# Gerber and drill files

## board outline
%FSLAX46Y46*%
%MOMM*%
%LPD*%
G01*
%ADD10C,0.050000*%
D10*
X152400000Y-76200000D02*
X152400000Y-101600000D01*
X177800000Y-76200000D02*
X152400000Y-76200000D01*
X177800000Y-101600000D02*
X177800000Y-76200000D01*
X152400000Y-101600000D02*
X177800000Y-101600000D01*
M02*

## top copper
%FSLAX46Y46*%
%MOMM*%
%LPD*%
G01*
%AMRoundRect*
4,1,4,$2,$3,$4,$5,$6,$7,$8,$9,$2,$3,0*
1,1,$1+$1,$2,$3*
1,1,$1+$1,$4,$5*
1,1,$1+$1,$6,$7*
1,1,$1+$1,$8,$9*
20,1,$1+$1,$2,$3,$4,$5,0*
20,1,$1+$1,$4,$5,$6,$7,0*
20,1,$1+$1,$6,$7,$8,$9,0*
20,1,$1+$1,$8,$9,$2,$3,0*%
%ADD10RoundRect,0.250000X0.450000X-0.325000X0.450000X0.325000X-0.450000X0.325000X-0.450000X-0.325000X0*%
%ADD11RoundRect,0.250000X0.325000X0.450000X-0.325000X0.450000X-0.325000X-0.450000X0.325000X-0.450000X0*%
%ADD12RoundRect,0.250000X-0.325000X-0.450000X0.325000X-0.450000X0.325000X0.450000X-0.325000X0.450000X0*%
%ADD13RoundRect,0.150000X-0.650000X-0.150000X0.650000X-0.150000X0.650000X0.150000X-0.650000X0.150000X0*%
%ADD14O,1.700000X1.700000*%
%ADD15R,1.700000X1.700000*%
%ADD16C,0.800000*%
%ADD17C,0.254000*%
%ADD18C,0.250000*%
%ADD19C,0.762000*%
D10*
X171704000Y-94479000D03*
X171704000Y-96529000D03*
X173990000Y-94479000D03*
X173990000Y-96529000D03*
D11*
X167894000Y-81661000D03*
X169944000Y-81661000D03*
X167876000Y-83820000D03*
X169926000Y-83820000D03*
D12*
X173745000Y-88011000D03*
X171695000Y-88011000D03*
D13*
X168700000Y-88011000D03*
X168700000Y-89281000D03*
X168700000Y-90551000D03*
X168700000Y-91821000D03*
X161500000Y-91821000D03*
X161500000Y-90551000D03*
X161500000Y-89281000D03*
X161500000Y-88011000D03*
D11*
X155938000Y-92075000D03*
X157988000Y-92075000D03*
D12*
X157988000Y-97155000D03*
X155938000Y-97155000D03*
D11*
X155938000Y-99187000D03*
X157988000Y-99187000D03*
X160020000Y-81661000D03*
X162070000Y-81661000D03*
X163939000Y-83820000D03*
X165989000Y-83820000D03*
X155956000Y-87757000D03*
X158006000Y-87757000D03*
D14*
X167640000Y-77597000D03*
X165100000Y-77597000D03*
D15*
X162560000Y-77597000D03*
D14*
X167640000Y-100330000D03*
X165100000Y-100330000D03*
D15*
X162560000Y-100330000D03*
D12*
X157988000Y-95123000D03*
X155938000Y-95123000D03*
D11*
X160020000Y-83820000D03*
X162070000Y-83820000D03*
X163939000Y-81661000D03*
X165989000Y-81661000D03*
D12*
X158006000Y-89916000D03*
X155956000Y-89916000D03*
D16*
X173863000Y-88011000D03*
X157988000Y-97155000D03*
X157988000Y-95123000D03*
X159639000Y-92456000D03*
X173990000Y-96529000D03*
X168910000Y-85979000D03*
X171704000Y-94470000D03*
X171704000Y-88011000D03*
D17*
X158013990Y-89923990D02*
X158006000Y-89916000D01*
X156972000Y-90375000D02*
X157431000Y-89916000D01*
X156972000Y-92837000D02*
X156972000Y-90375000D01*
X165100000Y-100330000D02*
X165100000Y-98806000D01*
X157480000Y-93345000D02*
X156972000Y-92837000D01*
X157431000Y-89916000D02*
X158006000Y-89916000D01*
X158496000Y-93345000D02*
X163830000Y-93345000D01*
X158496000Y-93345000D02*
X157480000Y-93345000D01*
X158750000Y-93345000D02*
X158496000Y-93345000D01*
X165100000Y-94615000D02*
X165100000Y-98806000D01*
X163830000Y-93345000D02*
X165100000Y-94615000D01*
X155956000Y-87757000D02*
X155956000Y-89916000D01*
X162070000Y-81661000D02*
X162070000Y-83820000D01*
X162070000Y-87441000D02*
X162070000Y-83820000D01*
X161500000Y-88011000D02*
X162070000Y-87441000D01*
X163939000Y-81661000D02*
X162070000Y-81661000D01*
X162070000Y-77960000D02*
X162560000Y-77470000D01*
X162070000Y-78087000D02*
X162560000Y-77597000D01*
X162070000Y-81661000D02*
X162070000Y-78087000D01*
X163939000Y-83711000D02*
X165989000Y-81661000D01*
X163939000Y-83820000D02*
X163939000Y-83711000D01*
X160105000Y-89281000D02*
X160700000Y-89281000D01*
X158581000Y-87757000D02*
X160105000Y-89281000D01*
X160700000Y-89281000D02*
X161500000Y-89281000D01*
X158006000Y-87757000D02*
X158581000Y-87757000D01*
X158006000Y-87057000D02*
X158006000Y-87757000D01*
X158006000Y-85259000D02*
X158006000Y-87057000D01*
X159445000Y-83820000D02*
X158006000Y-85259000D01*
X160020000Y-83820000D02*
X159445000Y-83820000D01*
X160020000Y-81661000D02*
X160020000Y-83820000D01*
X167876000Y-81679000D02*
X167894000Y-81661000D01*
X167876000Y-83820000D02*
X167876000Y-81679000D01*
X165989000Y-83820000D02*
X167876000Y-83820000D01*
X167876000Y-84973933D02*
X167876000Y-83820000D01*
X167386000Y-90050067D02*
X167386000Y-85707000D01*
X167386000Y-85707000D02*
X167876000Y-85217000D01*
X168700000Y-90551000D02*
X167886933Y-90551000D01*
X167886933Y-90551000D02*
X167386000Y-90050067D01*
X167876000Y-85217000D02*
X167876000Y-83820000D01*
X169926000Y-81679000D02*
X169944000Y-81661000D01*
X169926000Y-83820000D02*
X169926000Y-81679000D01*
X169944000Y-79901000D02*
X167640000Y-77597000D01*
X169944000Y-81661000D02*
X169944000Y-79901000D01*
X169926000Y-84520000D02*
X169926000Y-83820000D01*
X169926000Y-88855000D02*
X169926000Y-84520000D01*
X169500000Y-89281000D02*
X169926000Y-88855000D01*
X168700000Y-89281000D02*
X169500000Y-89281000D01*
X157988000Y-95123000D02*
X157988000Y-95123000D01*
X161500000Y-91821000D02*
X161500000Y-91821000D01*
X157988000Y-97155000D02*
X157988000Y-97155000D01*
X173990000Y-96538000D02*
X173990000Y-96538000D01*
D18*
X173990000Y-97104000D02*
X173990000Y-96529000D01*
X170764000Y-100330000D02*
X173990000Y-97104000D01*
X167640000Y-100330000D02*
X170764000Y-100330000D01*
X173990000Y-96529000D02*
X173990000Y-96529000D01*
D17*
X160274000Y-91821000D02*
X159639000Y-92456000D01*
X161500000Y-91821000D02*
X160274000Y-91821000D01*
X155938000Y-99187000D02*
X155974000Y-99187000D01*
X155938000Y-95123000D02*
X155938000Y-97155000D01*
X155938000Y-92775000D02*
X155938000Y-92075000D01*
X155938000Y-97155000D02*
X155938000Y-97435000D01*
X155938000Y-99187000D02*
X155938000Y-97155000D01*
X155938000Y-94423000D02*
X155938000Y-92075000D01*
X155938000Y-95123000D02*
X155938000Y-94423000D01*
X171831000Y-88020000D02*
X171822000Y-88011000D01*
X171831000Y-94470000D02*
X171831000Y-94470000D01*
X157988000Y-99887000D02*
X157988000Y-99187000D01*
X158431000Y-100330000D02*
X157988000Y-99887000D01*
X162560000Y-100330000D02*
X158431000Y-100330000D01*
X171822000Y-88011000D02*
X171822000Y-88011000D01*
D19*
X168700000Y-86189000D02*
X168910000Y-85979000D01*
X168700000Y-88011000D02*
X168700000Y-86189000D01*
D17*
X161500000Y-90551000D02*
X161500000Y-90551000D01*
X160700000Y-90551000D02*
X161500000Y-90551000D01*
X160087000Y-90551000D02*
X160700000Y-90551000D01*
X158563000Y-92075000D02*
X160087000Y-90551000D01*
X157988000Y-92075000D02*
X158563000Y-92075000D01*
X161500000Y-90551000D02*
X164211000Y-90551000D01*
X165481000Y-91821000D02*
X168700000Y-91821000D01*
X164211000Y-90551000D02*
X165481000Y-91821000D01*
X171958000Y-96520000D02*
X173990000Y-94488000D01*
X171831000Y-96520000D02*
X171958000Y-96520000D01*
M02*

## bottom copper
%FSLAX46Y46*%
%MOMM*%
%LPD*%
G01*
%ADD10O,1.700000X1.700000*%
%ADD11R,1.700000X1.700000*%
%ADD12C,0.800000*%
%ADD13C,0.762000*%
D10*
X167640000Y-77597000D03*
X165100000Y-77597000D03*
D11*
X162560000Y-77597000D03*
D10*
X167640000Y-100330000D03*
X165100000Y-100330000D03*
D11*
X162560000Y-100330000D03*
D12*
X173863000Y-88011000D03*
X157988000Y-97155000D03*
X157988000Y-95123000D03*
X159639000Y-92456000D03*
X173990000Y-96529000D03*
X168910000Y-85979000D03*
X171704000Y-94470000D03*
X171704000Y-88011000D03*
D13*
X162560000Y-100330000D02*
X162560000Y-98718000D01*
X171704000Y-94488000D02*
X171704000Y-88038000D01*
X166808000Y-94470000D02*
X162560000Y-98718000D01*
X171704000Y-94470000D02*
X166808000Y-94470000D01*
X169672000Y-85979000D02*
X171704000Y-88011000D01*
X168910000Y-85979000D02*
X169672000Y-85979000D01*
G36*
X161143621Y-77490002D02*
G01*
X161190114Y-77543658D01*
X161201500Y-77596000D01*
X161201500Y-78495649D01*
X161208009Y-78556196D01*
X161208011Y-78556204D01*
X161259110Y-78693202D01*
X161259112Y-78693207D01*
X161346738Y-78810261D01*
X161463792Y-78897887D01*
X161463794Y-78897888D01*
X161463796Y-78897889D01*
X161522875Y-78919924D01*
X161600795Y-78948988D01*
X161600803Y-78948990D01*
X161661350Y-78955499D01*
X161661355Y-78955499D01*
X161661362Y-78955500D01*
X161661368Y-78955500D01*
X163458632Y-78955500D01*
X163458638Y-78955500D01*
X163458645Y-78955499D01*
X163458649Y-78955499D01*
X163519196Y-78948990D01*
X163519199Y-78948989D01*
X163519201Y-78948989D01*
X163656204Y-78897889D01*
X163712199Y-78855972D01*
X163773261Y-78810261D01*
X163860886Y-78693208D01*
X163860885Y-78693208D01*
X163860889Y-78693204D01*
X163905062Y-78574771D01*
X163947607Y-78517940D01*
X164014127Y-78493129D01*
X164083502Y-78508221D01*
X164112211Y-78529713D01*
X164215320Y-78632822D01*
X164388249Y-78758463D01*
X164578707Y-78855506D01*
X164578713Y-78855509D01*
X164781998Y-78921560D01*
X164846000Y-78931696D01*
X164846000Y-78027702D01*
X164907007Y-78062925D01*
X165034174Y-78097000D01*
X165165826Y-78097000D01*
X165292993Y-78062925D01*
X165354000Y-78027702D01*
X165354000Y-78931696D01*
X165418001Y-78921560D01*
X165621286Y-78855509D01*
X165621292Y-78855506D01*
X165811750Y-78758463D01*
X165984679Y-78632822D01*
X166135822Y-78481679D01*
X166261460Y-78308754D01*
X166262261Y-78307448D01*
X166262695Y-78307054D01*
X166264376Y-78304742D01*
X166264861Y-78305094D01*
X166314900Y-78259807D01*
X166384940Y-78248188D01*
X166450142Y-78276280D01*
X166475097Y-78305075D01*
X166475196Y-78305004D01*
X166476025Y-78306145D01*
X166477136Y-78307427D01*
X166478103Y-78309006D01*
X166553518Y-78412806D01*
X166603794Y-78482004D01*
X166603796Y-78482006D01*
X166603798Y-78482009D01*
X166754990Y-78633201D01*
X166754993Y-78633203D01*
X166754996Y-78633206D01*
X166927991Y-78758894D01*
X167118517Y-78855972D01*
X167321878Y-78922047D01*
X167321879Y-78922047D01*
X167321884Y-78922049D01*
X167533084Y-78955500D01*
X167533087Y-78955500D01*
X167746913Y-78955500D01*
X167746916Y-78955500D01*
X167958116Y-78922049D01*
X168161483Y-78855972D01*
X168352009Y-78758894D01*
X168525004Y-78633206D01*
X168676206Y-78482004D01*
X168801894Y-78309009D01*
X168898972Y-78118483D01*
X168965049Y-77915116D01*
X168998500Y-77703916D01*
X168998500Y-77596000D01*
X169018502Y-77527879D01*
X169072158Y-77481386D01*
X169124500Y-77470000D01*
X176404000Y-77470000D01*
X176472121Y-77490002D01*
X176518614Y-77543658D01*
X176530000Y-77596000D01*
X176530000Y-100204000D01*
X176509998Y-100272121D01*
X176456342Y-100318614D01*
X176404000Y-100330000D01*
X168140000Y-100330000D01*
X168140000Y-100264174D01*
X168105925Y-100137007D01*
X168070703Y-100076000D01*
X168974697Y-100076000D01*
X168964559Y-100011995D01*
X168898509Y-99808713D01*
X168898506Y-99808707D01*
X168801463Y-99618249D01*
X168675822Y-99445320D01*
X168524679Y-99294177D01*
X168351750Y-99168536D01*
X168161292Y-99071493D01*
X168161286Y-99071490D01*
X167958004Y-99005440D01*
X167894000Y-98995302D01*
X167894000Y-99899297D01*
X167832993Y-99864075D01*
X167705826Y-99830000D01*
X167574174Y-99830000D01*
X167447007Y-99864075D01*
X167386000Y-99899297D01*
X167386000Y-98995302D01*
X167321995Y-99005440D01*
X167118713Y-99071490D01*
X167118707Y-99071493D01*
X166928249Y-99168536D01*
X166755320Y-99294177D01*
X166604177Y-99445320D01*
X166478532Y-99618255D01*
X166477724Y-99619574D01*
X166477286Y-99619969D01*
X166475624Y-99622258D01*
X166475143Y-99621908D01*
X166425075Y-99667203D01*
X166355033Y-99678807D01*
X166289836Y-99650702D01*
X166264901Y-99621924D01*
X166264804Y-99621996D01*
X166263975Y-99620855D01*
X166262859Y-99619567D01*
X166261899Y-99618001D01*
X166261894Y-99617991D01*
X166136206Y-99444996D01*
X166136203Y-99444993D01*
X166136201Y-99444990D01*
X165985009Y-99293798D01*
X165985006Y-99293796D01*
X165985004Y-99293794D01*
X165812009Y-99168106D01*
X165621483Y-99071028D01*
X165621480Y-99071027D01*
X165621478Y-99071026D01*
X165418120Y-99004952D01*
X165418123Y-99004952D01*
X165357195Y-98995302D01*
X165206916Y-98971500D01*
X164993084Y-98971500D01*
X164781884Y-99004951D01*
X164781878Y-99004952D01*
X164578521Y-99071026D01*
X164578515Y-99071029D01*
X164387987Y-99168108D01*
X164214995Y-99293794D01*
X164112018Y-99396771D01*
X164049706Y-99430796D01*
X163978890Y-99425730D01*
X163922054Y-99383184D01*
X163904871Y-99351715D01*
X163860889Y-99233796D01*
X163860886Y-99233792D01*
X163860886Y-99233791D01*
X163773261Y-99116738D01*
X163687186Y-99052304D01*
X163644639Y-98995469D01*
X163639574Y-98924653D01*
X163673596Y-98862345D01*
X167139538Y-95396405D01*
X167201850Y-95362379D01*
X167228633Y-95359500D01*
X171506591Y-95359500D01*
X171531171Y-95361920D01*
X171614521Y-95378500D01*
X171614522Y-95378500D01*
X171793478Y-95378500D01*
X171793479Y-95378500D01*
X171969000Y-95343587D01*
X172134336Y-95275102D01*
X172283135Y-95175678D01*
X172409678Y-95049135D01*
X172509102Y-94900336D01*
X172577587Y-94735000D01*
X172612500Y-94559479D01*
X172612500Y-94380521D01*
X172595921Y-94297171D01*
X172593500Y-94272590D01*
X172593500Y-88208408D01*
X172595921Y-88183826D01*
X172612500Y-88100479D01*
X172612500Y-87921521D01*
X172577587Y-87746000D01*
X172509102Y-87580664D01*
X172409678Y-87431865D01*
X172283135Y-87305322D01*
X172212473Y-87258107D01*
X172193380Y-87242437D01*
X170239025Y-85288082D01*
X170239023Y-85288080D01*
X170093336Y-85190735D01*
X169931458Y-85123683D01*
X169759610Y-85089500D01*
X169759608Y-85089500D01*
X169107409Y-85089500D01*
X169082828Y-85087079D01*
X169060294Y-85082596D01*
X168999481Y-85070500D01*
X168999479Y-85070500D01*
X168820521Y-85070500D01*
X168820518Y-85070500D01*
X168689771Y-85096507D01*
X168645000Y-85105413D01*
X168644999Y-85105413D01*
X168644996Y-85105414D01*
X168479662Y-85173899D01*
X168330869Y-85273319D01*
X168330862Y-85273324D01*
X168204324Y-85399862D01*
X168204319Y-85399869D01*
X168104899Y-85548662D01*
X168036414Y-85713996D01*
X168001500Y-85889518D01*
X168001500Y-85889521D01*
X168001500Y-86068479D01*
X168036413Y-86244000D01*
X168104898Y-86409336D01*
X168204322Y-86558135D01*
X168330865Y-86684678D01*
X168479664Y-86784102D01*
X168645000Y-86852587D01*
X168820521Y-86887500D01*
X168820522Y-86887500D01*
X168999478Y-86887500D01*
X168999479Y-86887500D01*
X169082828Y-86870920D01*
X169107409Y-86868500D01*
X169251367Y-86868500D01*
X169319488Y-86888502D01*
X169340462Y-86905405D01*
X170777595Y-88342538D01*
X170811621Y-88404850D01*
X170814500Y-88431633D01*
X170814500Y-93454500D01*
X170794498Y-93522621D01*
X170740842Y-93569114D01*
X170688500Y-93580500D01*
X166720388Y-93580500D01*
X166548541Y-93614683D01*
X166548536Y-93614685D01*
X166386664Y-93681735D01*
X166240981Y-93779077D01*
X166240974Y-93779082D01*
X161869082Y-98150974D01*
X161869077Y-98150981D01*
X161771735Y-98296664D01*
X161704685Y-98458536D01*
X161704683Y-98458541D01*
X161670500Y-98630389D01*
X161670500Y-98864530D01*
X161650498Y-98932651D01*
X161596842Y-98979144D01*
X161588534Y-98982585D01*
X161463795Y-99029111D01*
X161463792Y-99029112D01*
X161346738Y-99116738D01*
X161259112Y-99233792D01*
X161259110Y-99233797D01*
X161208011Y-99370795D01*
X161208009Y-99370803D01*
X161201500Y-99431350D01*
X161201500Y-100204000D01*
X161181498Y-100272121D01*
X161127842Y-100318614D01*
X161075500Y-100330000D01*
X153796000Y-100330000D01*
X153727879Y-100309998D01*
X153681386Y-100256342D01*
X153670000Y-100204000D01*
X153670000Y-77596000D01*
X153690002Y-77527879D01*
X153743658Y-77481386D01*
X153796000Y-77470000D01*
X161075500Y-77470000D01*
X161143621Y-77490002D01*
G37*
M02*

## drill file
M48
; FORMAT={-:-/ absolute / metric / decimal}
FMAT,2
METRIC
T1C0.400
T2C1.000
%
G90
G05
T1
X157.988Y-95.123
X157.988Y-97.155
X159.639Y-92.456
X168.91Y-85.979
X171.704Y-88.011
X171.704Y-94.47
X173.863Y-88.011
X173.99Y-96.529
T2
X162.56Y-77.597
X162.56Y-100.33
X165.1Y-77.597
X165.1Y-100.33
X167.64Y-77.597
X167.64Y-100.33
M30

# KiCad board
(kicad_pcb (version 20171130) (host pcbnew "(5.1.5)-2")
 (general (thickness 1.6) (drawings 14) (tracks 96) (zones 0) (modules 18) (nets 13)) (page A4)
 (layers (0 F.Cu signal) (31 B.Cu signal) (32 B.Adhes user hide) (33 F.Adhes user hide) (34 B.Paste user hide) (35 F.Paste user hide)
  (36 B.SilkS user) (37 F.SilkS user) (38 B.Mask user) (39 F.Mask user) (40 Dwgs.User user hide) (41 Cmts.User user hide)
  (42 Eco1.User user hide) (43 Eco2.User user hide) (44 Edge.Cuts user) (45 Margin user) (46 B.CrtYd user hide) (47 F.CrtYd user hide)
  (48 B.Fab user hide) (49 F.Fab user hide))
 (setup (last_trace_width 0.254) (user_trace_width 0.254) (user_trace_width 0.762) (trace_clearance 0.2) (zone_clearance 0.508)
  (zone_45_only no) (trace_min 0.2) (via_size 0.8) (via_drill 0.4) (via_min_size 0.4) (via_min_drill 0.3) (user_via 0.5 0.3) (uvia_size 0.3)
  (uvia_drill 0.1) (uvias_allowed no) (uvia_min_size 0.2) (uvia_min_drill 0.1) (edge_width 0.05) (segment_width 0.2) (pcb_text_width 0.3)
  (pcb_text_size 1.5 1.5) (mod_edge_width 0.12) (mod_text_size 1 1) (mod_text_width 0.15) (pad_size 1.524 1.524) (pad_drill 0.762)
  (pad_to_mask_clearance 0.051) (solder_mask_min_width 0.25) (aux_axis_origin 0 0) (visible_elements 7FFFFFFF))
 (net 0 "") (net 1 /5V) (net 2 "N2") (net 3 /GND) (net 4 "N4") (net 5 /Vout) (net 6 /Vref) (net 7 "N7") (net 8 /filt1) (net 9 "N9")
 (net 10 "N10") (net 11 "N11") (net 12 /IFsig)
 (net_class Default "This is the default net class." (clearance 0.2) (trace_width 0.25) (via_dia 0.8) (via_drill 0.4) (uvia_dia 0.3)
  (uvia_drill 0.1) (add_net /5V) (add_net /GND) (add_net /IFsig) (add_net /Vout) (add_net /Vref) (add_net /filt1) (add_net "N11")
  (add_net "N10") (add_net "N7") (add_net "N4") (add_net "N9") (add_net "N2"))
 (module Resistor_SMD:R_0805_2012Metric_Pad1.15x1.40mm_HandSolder (layer F.Cu) (at 171.704 95.504 90)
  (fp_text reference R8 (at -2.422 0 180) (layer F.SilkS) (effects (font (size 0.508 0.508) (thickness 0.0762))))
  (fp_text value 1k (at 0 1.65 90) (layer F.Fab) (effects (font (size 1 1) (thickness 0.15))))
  (pad 2 smd roundrect (at 1.025 0 90) (size 1.15 1.4) (layers F.Cu F.Paste F.Mask) (roundrect_rratio 0.217391) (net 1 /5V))
  (pad 1 smd roundrect (at -1.025 0 90) (size 1.15 1.4) (layers F.Cu F.Paste F.Mask) (roundrect_rratio 0.217391) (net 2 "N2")))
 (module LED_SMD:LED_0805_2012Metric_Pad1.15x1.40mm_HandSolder (layer F.Cu) (at 173.99 95.504 90)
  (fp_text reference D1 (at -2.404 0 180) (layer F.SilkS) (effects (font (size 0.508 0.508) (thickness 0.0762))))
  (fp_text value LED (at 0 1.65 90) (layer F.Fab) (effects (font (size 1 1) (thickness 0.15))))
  (pad 2 smd roundrect (at 1.025 0 90) (size 1.15 1.4) (layers F.Cu F.Paste F.Mask) (roundrect_rratio 0.217391) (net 2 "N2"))
  (pad 1 smd roundrect (at -1.025 0 90) (size 1.15 1.4) (layers F.Cu F.Paste F.Mask) (roundrect_rratio 0.217391) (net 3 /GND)))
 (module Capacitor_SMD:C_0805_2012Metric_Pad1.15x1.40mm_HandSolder (layer F.Cu) (at 168.919 81.661 180)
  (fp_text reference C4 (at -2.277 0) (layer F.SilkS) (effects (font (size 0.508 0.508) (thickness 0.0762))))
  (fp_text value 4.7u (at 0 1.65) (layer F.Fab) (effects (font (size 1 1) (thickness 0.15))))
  (pad 2 smd roundrect (at 1.025 0 180) (size 1.15 1.4) (layers F.Cu F.Paste F.Mask) (roundrect_rratio 0.217391) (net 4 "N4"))
  (pad 1 smd roundrect (at -1.025 0 180) (size 1.15 1.4) (layers F.Cu F.Paste F.Mask) (roundrect_rratio 0.217391) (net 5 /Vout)))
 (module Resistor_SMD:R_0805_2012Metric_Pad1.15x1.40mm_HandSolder (layer F.Cu) (at 168.901 83.82 180)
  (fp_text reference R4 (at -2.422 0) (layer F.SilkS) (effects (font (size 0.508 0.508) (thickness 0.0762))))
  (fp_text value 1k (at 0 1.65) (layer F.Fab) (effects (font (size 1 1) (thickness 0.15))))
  (pad 2 smd roundrect (at 1.025 0 180) (size 1.15 1.4) (layers F.Cu F.Paste F.Mask) (roundrect_rratio 0.217391) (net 4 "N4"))
  (pad 1 smd roundrect (at -1.025 0 180) (size 1.15 1.4) (layers F.Cu F.Paste F.Mask) (roundrect_rratio 0.217391) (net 5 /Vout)))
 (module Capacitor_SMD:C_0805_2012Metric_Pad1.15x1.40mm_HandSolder (layer F.Cu) (at 172.72 88.011)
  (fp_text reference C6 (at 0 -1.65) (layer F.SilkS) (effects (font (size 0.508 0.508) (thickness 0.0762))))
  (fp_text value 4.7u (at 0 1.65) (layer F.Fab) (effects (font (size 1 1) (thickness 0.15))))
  (pad 2 smd roundrect (at 1.025 0) (size 1.15 1.4) (layers F.Cu F.Paste F.Mask) (roundrect_rratio 0.217391) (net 3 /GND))
  (pad 1 smd roundrect (at -1.025 0) (size 1.15 1.4) (layers F.Cu F.Paste F.Mask) (roundrect_rratio 0.217391) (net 1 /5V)))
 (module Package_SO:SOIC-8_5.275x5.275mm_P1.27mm (layer F.Cu) (at 165.1 89.916)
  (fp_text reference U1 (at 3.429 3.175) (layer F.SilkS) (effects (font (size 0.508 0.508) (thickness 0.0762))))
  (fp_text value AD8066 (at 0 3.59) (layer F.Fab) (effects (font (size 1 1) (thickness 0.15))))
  (pad 8 smd roundrect (at 3.6 -1.905) (size 1.6 0.6) (layers F.Cu F.Paste F.Mask) (roundrect_rratio 0.25) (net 1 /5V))
  (pad 7 smd roundrect (at 3.6 -0.635) (size 1.6 0.6) (layers F.Cu F.Paste F.Mask) (roundrect_rratio 0.25) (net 5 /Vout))
  (pad 6 smd roundrect (at 3.6 0.635) (size 1.6 0.6) (layers F.Cu F.Paste F.Mask) (roundrect_rratio 0.25) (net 4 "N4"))
  (pad 5 smd roundrect (at 3.6 1.905) (size 1.6 0.6) (layers F.Cu F.Paste F.Mask) (roundrect_rratio 0.25) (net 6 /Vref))
  (pad 4 smd roundrect (at -3.6 1.905) (size 1.6 0.6) (layers F.Cu F.Paste F.Mask) (roundrect_rratio 0.25) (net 3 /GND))
  (pad 3 smd roundrect (at -3.6 0.635) (size 1.6 0.6) (layers F.Cu F.Paste F.Mask) (roundrect_rratio 0.25) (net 6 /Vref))
  (pad 2 smd roundrect (at -3.6 -0.635) (size 1.6 0.6) (layers F.Cu F.Paste F.Mask) (roundrect_rratio 0.25) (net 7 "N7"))
  (pad 1 smd roundrect (at -3.6 -1.905) (size 1.6 0.6) (layers F.Cu F.Paste F.Mask) (roundrect_rratio 0.25) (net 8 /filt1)))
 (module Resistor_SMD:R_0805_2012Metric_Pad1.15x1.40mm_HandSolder (layer F.Cu) (at 156.963 92.075 180)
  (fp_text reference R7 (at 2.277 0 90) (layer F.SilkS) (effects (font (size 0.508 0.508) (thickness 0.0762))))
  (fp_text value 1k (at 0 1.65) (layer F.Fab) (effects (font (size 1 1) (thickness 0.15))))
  (pad 2 smd roundrect (at 1.025 0 180) (size 1.15 1.4) (layers F.Cu F.Paste F.Mask) (roundrect_rratio 0.217391) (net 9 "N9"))
  (pad 1 smd roundrect (at -1.025 0 180) (size 1.15 1.4) (layers F.Cu F.Paste F.Mask) (roundrect_rratio 0.217391) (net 6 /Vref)))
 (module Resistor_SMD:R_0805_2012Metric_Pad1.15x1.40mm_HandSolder (layer F.Cu) (at 156.963 97.155)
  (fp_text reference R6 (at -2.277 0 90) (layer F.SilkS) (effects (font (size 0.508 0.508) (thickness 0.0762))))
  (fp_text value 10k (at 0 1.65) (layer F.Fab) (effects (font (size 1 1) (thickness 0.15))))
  (pad 2 smd roundrect (at 1.025 0) (size 1.15 1.4) (layers F.Cu F.Paste F.Mask) (roundrect_rratio 0.217391) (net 3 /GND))
  (pad 1 smd roundrect (at -1.025 0) (size 1.15 1.4) (layers F.Cu F.Paste F.Mask) (roundrect_rratio 0.217391) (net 9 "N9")))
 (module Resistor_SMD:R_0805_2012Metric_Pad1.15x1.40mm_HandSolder (layer F.Cu) (at 156.963 99.187 180)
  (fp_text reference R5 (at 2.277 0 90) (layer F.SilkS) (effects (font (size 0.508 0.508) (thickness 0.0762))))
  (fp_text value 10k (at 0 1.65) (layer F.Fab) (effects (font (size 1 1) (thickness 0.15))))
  (pad 2 smd roundrect (at 1.025 0 180) (size 1.15 1.4) (layers F.Cu F.Paste F.Mask) (roundrect_rratio 0.217391) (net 9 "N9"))
  (pad 1 smd roundrect (at -1.025 0 180) (size 1.15 1.4) (layers F.Cu F.Paste F.Mask) (roundrect_rratio 0.217391) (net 1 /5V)))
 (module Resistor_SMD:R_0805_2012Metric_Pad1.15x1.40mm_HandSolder (layer F.Cu) (at 161.045 81.661 180)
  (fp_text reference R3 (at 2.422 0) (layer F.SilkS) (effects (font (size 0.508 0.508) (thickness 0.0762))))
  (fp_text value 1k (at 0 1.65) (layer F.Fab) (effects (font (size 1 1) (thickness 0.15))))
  (pad 2 smd roundrect (at 1.025 0 180) (size 1.15 1.4) (layers F.Cu F.Paste F.Mask) (roundrect_rratio 0.217391) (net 7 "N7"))
  (pad 1 smd roundrect (at -1.025 0 180) (size 1.15 1.4) (layers F.Cu F.Paste F.Mask) (roundrect_rratio 0.217391) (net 8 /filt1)))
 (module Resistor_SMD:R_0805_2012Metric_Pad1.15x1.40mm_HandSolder (layer F.Cu) (at 164.964 83.82 180)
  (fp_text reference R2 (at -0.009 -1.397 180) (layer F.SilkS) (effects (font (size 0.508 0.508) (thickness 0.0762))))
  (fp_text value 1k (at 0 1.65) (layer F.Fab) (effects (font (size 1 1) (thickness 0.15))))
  (pad 2 smd roundrect (at 1.025 0 180) (size 1.15 1.4) (layers F.Cu F.Paste F.Mask) (roundrect_rratio 0.217391) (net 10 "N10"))
  (pad 1 smd roundrect (at -1.025 0 180) (size 1.15 1.4) (layers F.Cu F.Paste F.Mask) (roundrect_rratio 0.217391) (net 4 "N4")))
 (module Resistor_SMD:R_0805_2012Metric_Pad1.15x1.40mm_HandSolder (layer F.Cu) (at 156.981 87.757 180)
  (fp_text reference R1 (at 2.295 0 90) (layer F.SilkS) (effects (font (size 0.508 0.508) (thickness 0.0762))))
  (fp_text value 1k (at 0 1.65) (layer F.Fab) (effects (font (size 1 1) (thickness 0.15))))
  (pad 2 smd roundrect (at 1.025 0 180) (size 1.15 1.4) (layers F.Cu F.Paste F.Mask) (roundrect_rratio 0.217391) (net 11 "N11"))
  (pad 1 smd roundrect (at -1.025 0 180) (size 1.15 1.4) (layers F.Cu F.Paste F.Mask) (roundrect_rratio 0.217391) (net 7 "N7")))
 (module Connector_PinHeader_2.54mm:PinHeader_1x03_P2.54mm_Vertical (layer F.Cu) (at 162.56 77.597 90)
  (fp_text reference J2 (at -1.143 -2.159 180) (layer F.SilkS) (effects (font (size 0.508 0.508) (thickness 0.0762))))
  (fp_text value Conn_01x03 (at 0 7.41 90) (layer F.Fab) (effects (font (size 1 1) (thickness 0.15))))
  (pad 3 thru_hole oval (at 0 5.08 90) (size 1.7 1.7) (drill 1) (layers *.Cu *.Mask) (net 5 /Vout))
  (pad 2 thru_hole oval (at 0 2.54 90) (size 1.7 1.7) (drill 1) (layers *.Cu *.Mask) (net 3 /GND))
  (pad 1 thru_hole rect (at 0 0 90) (size 1.7 1.7) (drill 1) (layers *.Cu *.Mask) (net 8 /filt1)))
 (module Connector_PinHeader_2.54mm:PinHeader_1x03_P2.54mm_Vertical (layer F.Cu) (at 162.56 100.33 90)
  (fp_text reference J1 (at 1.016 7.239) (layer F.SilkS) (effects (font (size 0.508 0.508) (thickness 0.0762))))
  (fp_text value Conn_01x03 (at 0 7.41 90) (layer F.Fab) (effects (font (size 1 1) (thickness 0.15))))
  (pad 3 thru_hole oval (at 0 5.08 90) (size 1.7 1.7) (drill 1) (layers *.Cu *.Mask) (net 3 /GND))
  (pad 2 thru_hole oval (at 0 2.54 90) (size 1.7 1.7) (drill 1) (layers *.Cu *.Mask) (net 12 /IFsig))
  (pad 1 thru_hole rect (at 0 0 90) (size 1.7 1.7) (drill 1) (layers *.Cu *.Mask) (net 1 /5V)))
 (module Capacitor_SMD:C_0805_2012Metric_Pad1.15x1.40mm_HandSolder (layer F.Cu) (at 156.963 95.123)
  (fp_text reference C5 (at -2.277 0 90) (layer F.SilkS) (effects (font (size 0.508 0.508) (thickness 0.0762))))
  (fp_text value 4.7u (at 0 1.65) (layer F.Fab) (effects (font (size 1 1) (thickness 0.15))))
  (pad 2 smd roundrect (at 1.025 0) (size 1.15 1.4) (layers F.Cu F.Paste F.Mask) (roundrect_rratio 0.217391) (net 3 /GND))
  (pad 1 smd roundrect (at -1.025 0) (size 1.15 1.4) (layers F.Cu F.Paste F.Mask) (roundrect_rratio 0.217391) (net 9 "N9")))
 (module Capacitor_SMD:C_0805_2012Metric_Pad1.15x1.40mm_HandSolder (layer F.Cu) (at 161.045 83.82 180)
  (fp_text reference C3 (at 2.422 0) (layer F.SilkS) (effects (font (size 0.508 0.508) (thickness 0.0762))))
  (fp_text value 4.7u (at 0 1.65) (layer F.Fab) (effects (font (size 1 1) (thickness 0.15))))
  (pad 2 smd roundrect (at 1.025 0 180) (size 1.15 1.4) (layers F.Cu F.Paste F.Mask) (roundrect_rratio 0.217391) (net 7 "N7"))
  (pad 1 smd roundrect (at -1.025 0 180) (size 1.15 1.4) (layers F.Cu F.Paste F.Mask) (roundrect_rratio 0.217391) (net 8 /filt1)))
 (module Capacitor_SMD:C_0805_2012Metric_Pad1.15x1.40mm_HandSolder (layer F.Cu) (at 164.964 81.661 180)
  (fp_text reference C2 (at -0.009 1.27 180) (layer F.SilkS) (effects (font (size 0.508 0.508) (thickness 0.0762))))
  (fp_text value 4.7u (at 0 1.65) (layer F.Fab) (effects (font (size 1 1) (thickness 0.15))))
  (pad 2 smd roundrect (at 1.025 0 180) (size 1.15 1.4) (layers F.Cu F.Paste F.Mask) (roundrect_rratio 0.217391) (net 8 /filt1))
  (pad 1 smd roundrect (at -1.025 0 180) (size 1.15 1.4) (layers F.Cu F.Paste F.Mask) (roundrect_rratio 0.217391) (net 10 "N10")))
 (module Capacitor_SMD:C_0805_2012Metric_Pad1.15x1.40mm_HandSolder (layer F.Cu) (at 156.981 89.916)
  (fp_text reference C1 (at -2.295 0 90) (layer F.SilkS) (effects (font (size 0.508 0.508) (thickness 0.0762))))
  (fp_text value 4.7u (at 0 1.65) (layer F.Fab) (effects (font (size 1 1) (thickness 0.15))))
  (pad 2 smd roundrect (at 1.025 0) (size 1.15 1.4) (layers F.Cu F.Paste F.Mask) (roundrect_rratio 0.217391) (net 12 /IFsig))
  (pad 1 smd roundrect (at -1.025 0) (size 1.15 1.4) (layers F.Cu F.Paste F.Mask) (roundrect_rratio 0.217391) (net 11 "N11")))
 (gr_line (start 152.4 76.2) (end 152.4 101.6) (layer Edge.Cuts) (width 0.05))
 (gr_line (start 177.8 76.2) (end 152.4 76.2) (layer Edge.Cuts) (width 0.05))
 (gr_line (start 177.8 101.6) (end 177.8 76.2) (layer Edge.Cuts) (width 0.05))
 (gr_line (start 152.4 101.6) (end 177.8 101.6) (layer Edge.Cuts) (width 0.05))
 (segment (start 158.01399 89.92399) (end 158.006 89.916) (width 0.254) (layer F.Cu) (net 12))
 (segment (start 156.972 90.375) (end 157.431 89.916) (width 0.254) (layer F.Cu) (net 12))
 (segment (start 156.972 92.837) (end 156.972 90.375) (width 0.254) (layer F.Cu) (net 12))
 (segment (start 165.1 100.33) (end 165.1 98.806) (width 0.254) (layer F.Cu) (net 12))
 (segment (start 157.48 93.345) (end 156.972 92.837) (width 0.254) (layer F.Cu) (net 12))
 (segment (start 157.431 89.916) (end 158.006 89.916) (width 0.254) (layer F.Cu) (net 12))
 (segment (start 158.496 93.345) (end 163.83 93.345) (width 0.254) (layer F.Cu) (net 12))
 (segment (start 158.496 93.345) (end 157.48 93.345) (width 0.254) (layer F.Cu) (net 12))
 (segment (start 158.75 93.345) (end 158.496 93.345) (width 0.254) (layer F.Cu) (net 12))
 (segment (start 165.1 94.615) (end 165.1 98.806) (width 0.254) (layer F.Cu) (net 12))
 (segment (start 163.83 93.345) (end 165.1 94.615) (width 0.254) (layer F.Cu) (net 12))
 (segment (start 155.956 87.757) (end 155.956 89.916) (width 0.254) (layer F.Cu) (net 11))
 (segment (start 162.07 81.661) (end 162.07 83.82) (width 0.254) (layer F.Cu) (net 8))
 (segment (start 162.07 87.441) (end 162.07 83.82) (width 0.254) (layer F.Cu) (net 8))
 (segment (start 161.5 88.011) (end 162.07 87.441) (width 0.254) (layer F.Cu) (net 8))
 (segment (start 163.939 81.661) (end 162.07 81.661) (width 0.254) (layer F.Cu) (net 8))
 (segment (start 162.07 77.96) (end 162.56 77.47) (width 0.254) (layer F.Cu) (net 8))
 (segment (start 162.07 78.087) (end 162.56 77.597) (width 0.254) (layer F.Cu) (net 8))
 (segment (start 162.07 81.661) (end 162.07 78.087) (width 0.254) (layer F.Cu) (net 8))
 (segment (start 163.939 83.711) (end 165.989 81.661) (width 0.254) (layer F.Cu) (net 10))
 (segment (start 163.939 83.82) (end 163.939 83.711) (width 0.254) (layer F.Cu) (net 10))
 (segment (start 160.105 89.281) (end 160.7 89.281) (width 0.254) (layer F.Cu) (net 7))
 (segment (start 158.581 87.757) (end 160.105 89.281) (width 0.254) (layer F.Cu) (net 7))
 (segment (start 160.7 89.281) (end 161.5 89.281) (width 0.254) (layer F.Cu) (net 7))
 (segment (start 158.006 87.757) (end 158.581 87.757) (width 0.254) (layer F.Cu) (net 7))
 (segment (start 158.006 87.057) (end 158.006 87.757) (width 0.254) (layer F.Cu) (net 7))
 (segment (start 158.006 85.259) (end 158.006 87.057) (width 0.254) (layer F.Cu) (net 7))
 (segment (start 159.445 83.82) (end 158.006 85.259) (width 0.254) (layer F.Cu) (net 7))
 (segment (start 160.02 83.82) (end 159.445 83.82) (width 0.254) (layer F.Cu) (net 7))
 (segment (start 160.02 81.661) (end 160.02 83.82) (width 0.254) (layer F.Cu) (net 7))
 (segment (start 167.876 81.679) (end 167.894 81.661) (width 0.254) (layer F.Cu) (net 4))
 (segment (start 167.876 83.82) (end 167.876 81.679) (width 0.254) (layer F.Cu) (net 4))
 (segment (start 165.989 83.82) (end 167.876 83.82) (width 0.254) (layer F.Cu) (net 4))
 (segment (start 167.876 84.973933) (end 167.876 83.82) (width 0.254) (layer F.Cu) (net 4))
 (segment (start 167.386 90.050067) (end 167.386 85.707) (width 0.254) (layer F.Cu) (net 4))
 (segment (start 167.386 85.707) (end 167.876 85.217) (width 0.254) (layer F.Cu) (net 4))
 (segment (start 168.7 90.551) (end 167.886933 90.551) (width 0.254) (layer F.Cu) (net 4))
 (segment (start 167.886933 90.551) (end 167.386 90.050067) (width 0.254) (layer F.Cu) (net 4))
 (segment (start 167.876 85.217) (end 167.876 83.82) (width 0.254) (layer F.Cu) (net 4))
 (segment (start 169.926 81.679) (end 169.944 81.661) (width 0.254) (layer F.Cu) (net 5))
 (segment (start 169.926 83.82) (end 169.926 81.679) (width 0.254) (layer F.Cu) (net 5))
 (segment (start 169.944 79.901) (end 167.64 77.597) (width 0.254) (layer F.Cu) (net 5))
 (segment (start 169.944 81.661) (end 169.944 79.901) (width 0.254) (layer F.Cu) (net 5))
 (segment (start 169.926 84.52) (end 169.926 83.82) (width 0.254) (layer F.Cu) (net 5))
 (segment (start 169.926 88.855) (end 169.926 84.52) (width 0.254) (layer F.Cu) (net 5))
 (segment (start 169.5 89.281) (end 169.926 88.855) (width 0.254) (layer F.Cu) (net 5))
 (segment (start 168.7 89.281) (end 169.5 89.281) (width 0.254) (layer F.Cu) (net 5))
 (via (at 173.863 88.011) (size 0.8) (drill 0.4) (layers F.Cu B.Cu) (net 3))
 (segment (start 157.988 95.123) (end 157.988 95.123) (width 0.254) (layer F.Cu) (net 3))
 (segment (start 161.5 91.821) (end 161.5 91.821) (width 0.254) (layer F.Cu) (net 3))
 (segment (start 157.988 97.155) (end 157.988 97.155) (width 0.254) (layer F.Cu) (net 3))
 (via (at 157.988 97.155) (size 0.8) (drill 0.4) (layers F.Cu B.Cu) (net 3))
 (via (at 157.988 95.123) (size 0.8) (drill 0.4) (layers F.Cu B.Cu) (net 3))
 (segment (start 173.99 96.538) (end 173.99 96.538) (width 0.254) (layer F.Cu) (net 3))
 (via (at 159.639 92.456) (size 0.8) (drill 0.4) (layers F.Cu B.Cu) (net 3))
 (segment (start 173.99 97.104) (end 173.99 96.529) (width 0.25) (layer F.Cu) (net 3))
 (segment (start 170.764 100.33) (end 173.99 97.104) (width 0.25) (layer F.Cu) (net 3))
 (segment (start 167.64 100.33) (end 170.764 100.33) (width 0.25) (layer F.Cu) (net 3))
 (segment (start 173.99 96.529) (end 173.99 96.529) (width 0.25) (layer F.Cu) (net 3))
 (via (at 173.99 96.529) (size 0.8) (drill 0.4) (layers F.Cu B.Cu) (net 3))
 (segment (start 160.274 91.821) (end 159.639 92.456) (width 0.254) (layer F.Cu) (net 3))
 (segment (start 161.5 91.821) (end 160.274 91.821) (width 0.254) (layer F.Cu) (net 3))
 (segment (start 155.938 99.187) (end 155.974 99.187) (width 0.254) (layer F.Cu) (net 9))
 (segment (start 155.938 95.123) (end 155.938 97.155) (width 0.254) (layer F.Cu) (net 9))
 (segment (start 155.938 92.775) (end 155.938 92.075) (width 0.254) (layer F.Cu) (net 9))
 (segment (start 155.938 97.155) (end 155.938 97.435) (width 0.254) (layer F.Cu) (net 9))
 (segment (start 155.938 99.187) (end 155.938 97.155) (width 0.254) (layer F.Cu) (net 9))
 (segment (start 155.938 94.423) (end 155.938 92.075) (width 0.254) (layer F.Cu) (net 9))
 (segment (start 155.938 95.123) (end 155.938 94.423) (width 0.254) (layer F.Cu) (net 9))
 (via (at 168.91 85.979) (size 0.8) (drill 0.4) (layers F.Cu B.Cu) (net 1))
 (segment (start 171.831 88.02) (end 171.822 88.011) (width 0.254) (layer F.Cu) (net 1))
 (segment (start 171.831 94.47) (end 171.831 94.47) (width 0.254) (layer F.Cu) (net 1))
 (segment (start 157.988 99.887) (end 157.988 99.187) (width 0.254) (layer F.Cu) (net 1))
 (segment (start 158.431 100.33) (end 157.988 99.887) (width 0.254) (layer F.Cu) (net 1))
 (segment (start 162.56 100.33) (end 158.431 100.33) (width 0.254) (layer F.Cu) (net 1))
 (via (at 171.704 94.47) (size 0.8) (drill 0.4) (layers F.Cu B.Cu) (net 1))
 (segment (start 162.56 100.33) (end 162.56 98.718) (width 0.762) (layer B.Cu) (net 1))
 (segment (start 171.822 88.011) (end 171.822 88.011) (width 0.254) (layer F.Cu) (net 1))
 (via (at 171.704 88.011) (size 0.8) (drill 0.4) (layers F.Cu B.Cu) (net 1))
 (segment (start 171.704 94.488) (end 171.704 88.038) (width 0.762) (layer B.Cu) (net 1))
 (segment (start 166.808 94.47) (end 162.56 98.718) (width 0.762) (layer B.Cu) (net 1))
 (segment (start 171.704 94.47) (end 166.808 94.47) (width 0.762) (layer B.Cu) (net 1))
 (segment (start 168.7 86.189) (end 168.91 85.979) (width 0.762) (layer F.Cu) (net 1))
 (segment (start 168.7 88.011) (end 168.7 86.189) (width 0.762) (layer F.Cu) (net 1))
 (segment (start 169.672 85.979) (end 171.704 88.011) (width 0.762) (layer B.Cu) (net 1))
 (segment (start 168.91 85.979) (end 169.672 85.979) (width 0.762) (layer B.Cu) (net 1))
 (segment (start 161.5 90.551) (end 161.5 90.551) (width 0.254) (layer F.Cu) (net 6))
 (segment (start 160.7 90.551) (end 161.5 90.551) (width 0.254) (layer F.Cu) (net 6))
 (segment (start 160.087 90.551) (end 160.7 90.551) (width 0.254) (layer F.Cu) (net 6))
 (segment (start 158.563 92.075) (end 160.087 90.551) (width 0.254) (layer F.Cu) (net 6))
 (segment (start 157.988 92.075) (end 158.563 92.075) (width 0.254) (layer F.Cu) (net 6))
 (segment (start 161.5 90.551) (end 164.211 90.551) (width 0.254) (layer F.Cu) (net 6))
 (segment (start 165.481 91.821) (end 168.7 91.821) (width 0.254) (layer F.Cu) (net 6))
 (segment (start 164.211 90.551) (end 165.481 91.821) (width 0.254) (layer F.Cu) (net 6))
 (segment (start 171.958 96.52) (end 173.99 94.488) (width 0.254) (layer F.Cu) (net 2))
 (segment (start 171.831 96.52) (end 171.958 96.52) (width 0.254) (layer F.Cu) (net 2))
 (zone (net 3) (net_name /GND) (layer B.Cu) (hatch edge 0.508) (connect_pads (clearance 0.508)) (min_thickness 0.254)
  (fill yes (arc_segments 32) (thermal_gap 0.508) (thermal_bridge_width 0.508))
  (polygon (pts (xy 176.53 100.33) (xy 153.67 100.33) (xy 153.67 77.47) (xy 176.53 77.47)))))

